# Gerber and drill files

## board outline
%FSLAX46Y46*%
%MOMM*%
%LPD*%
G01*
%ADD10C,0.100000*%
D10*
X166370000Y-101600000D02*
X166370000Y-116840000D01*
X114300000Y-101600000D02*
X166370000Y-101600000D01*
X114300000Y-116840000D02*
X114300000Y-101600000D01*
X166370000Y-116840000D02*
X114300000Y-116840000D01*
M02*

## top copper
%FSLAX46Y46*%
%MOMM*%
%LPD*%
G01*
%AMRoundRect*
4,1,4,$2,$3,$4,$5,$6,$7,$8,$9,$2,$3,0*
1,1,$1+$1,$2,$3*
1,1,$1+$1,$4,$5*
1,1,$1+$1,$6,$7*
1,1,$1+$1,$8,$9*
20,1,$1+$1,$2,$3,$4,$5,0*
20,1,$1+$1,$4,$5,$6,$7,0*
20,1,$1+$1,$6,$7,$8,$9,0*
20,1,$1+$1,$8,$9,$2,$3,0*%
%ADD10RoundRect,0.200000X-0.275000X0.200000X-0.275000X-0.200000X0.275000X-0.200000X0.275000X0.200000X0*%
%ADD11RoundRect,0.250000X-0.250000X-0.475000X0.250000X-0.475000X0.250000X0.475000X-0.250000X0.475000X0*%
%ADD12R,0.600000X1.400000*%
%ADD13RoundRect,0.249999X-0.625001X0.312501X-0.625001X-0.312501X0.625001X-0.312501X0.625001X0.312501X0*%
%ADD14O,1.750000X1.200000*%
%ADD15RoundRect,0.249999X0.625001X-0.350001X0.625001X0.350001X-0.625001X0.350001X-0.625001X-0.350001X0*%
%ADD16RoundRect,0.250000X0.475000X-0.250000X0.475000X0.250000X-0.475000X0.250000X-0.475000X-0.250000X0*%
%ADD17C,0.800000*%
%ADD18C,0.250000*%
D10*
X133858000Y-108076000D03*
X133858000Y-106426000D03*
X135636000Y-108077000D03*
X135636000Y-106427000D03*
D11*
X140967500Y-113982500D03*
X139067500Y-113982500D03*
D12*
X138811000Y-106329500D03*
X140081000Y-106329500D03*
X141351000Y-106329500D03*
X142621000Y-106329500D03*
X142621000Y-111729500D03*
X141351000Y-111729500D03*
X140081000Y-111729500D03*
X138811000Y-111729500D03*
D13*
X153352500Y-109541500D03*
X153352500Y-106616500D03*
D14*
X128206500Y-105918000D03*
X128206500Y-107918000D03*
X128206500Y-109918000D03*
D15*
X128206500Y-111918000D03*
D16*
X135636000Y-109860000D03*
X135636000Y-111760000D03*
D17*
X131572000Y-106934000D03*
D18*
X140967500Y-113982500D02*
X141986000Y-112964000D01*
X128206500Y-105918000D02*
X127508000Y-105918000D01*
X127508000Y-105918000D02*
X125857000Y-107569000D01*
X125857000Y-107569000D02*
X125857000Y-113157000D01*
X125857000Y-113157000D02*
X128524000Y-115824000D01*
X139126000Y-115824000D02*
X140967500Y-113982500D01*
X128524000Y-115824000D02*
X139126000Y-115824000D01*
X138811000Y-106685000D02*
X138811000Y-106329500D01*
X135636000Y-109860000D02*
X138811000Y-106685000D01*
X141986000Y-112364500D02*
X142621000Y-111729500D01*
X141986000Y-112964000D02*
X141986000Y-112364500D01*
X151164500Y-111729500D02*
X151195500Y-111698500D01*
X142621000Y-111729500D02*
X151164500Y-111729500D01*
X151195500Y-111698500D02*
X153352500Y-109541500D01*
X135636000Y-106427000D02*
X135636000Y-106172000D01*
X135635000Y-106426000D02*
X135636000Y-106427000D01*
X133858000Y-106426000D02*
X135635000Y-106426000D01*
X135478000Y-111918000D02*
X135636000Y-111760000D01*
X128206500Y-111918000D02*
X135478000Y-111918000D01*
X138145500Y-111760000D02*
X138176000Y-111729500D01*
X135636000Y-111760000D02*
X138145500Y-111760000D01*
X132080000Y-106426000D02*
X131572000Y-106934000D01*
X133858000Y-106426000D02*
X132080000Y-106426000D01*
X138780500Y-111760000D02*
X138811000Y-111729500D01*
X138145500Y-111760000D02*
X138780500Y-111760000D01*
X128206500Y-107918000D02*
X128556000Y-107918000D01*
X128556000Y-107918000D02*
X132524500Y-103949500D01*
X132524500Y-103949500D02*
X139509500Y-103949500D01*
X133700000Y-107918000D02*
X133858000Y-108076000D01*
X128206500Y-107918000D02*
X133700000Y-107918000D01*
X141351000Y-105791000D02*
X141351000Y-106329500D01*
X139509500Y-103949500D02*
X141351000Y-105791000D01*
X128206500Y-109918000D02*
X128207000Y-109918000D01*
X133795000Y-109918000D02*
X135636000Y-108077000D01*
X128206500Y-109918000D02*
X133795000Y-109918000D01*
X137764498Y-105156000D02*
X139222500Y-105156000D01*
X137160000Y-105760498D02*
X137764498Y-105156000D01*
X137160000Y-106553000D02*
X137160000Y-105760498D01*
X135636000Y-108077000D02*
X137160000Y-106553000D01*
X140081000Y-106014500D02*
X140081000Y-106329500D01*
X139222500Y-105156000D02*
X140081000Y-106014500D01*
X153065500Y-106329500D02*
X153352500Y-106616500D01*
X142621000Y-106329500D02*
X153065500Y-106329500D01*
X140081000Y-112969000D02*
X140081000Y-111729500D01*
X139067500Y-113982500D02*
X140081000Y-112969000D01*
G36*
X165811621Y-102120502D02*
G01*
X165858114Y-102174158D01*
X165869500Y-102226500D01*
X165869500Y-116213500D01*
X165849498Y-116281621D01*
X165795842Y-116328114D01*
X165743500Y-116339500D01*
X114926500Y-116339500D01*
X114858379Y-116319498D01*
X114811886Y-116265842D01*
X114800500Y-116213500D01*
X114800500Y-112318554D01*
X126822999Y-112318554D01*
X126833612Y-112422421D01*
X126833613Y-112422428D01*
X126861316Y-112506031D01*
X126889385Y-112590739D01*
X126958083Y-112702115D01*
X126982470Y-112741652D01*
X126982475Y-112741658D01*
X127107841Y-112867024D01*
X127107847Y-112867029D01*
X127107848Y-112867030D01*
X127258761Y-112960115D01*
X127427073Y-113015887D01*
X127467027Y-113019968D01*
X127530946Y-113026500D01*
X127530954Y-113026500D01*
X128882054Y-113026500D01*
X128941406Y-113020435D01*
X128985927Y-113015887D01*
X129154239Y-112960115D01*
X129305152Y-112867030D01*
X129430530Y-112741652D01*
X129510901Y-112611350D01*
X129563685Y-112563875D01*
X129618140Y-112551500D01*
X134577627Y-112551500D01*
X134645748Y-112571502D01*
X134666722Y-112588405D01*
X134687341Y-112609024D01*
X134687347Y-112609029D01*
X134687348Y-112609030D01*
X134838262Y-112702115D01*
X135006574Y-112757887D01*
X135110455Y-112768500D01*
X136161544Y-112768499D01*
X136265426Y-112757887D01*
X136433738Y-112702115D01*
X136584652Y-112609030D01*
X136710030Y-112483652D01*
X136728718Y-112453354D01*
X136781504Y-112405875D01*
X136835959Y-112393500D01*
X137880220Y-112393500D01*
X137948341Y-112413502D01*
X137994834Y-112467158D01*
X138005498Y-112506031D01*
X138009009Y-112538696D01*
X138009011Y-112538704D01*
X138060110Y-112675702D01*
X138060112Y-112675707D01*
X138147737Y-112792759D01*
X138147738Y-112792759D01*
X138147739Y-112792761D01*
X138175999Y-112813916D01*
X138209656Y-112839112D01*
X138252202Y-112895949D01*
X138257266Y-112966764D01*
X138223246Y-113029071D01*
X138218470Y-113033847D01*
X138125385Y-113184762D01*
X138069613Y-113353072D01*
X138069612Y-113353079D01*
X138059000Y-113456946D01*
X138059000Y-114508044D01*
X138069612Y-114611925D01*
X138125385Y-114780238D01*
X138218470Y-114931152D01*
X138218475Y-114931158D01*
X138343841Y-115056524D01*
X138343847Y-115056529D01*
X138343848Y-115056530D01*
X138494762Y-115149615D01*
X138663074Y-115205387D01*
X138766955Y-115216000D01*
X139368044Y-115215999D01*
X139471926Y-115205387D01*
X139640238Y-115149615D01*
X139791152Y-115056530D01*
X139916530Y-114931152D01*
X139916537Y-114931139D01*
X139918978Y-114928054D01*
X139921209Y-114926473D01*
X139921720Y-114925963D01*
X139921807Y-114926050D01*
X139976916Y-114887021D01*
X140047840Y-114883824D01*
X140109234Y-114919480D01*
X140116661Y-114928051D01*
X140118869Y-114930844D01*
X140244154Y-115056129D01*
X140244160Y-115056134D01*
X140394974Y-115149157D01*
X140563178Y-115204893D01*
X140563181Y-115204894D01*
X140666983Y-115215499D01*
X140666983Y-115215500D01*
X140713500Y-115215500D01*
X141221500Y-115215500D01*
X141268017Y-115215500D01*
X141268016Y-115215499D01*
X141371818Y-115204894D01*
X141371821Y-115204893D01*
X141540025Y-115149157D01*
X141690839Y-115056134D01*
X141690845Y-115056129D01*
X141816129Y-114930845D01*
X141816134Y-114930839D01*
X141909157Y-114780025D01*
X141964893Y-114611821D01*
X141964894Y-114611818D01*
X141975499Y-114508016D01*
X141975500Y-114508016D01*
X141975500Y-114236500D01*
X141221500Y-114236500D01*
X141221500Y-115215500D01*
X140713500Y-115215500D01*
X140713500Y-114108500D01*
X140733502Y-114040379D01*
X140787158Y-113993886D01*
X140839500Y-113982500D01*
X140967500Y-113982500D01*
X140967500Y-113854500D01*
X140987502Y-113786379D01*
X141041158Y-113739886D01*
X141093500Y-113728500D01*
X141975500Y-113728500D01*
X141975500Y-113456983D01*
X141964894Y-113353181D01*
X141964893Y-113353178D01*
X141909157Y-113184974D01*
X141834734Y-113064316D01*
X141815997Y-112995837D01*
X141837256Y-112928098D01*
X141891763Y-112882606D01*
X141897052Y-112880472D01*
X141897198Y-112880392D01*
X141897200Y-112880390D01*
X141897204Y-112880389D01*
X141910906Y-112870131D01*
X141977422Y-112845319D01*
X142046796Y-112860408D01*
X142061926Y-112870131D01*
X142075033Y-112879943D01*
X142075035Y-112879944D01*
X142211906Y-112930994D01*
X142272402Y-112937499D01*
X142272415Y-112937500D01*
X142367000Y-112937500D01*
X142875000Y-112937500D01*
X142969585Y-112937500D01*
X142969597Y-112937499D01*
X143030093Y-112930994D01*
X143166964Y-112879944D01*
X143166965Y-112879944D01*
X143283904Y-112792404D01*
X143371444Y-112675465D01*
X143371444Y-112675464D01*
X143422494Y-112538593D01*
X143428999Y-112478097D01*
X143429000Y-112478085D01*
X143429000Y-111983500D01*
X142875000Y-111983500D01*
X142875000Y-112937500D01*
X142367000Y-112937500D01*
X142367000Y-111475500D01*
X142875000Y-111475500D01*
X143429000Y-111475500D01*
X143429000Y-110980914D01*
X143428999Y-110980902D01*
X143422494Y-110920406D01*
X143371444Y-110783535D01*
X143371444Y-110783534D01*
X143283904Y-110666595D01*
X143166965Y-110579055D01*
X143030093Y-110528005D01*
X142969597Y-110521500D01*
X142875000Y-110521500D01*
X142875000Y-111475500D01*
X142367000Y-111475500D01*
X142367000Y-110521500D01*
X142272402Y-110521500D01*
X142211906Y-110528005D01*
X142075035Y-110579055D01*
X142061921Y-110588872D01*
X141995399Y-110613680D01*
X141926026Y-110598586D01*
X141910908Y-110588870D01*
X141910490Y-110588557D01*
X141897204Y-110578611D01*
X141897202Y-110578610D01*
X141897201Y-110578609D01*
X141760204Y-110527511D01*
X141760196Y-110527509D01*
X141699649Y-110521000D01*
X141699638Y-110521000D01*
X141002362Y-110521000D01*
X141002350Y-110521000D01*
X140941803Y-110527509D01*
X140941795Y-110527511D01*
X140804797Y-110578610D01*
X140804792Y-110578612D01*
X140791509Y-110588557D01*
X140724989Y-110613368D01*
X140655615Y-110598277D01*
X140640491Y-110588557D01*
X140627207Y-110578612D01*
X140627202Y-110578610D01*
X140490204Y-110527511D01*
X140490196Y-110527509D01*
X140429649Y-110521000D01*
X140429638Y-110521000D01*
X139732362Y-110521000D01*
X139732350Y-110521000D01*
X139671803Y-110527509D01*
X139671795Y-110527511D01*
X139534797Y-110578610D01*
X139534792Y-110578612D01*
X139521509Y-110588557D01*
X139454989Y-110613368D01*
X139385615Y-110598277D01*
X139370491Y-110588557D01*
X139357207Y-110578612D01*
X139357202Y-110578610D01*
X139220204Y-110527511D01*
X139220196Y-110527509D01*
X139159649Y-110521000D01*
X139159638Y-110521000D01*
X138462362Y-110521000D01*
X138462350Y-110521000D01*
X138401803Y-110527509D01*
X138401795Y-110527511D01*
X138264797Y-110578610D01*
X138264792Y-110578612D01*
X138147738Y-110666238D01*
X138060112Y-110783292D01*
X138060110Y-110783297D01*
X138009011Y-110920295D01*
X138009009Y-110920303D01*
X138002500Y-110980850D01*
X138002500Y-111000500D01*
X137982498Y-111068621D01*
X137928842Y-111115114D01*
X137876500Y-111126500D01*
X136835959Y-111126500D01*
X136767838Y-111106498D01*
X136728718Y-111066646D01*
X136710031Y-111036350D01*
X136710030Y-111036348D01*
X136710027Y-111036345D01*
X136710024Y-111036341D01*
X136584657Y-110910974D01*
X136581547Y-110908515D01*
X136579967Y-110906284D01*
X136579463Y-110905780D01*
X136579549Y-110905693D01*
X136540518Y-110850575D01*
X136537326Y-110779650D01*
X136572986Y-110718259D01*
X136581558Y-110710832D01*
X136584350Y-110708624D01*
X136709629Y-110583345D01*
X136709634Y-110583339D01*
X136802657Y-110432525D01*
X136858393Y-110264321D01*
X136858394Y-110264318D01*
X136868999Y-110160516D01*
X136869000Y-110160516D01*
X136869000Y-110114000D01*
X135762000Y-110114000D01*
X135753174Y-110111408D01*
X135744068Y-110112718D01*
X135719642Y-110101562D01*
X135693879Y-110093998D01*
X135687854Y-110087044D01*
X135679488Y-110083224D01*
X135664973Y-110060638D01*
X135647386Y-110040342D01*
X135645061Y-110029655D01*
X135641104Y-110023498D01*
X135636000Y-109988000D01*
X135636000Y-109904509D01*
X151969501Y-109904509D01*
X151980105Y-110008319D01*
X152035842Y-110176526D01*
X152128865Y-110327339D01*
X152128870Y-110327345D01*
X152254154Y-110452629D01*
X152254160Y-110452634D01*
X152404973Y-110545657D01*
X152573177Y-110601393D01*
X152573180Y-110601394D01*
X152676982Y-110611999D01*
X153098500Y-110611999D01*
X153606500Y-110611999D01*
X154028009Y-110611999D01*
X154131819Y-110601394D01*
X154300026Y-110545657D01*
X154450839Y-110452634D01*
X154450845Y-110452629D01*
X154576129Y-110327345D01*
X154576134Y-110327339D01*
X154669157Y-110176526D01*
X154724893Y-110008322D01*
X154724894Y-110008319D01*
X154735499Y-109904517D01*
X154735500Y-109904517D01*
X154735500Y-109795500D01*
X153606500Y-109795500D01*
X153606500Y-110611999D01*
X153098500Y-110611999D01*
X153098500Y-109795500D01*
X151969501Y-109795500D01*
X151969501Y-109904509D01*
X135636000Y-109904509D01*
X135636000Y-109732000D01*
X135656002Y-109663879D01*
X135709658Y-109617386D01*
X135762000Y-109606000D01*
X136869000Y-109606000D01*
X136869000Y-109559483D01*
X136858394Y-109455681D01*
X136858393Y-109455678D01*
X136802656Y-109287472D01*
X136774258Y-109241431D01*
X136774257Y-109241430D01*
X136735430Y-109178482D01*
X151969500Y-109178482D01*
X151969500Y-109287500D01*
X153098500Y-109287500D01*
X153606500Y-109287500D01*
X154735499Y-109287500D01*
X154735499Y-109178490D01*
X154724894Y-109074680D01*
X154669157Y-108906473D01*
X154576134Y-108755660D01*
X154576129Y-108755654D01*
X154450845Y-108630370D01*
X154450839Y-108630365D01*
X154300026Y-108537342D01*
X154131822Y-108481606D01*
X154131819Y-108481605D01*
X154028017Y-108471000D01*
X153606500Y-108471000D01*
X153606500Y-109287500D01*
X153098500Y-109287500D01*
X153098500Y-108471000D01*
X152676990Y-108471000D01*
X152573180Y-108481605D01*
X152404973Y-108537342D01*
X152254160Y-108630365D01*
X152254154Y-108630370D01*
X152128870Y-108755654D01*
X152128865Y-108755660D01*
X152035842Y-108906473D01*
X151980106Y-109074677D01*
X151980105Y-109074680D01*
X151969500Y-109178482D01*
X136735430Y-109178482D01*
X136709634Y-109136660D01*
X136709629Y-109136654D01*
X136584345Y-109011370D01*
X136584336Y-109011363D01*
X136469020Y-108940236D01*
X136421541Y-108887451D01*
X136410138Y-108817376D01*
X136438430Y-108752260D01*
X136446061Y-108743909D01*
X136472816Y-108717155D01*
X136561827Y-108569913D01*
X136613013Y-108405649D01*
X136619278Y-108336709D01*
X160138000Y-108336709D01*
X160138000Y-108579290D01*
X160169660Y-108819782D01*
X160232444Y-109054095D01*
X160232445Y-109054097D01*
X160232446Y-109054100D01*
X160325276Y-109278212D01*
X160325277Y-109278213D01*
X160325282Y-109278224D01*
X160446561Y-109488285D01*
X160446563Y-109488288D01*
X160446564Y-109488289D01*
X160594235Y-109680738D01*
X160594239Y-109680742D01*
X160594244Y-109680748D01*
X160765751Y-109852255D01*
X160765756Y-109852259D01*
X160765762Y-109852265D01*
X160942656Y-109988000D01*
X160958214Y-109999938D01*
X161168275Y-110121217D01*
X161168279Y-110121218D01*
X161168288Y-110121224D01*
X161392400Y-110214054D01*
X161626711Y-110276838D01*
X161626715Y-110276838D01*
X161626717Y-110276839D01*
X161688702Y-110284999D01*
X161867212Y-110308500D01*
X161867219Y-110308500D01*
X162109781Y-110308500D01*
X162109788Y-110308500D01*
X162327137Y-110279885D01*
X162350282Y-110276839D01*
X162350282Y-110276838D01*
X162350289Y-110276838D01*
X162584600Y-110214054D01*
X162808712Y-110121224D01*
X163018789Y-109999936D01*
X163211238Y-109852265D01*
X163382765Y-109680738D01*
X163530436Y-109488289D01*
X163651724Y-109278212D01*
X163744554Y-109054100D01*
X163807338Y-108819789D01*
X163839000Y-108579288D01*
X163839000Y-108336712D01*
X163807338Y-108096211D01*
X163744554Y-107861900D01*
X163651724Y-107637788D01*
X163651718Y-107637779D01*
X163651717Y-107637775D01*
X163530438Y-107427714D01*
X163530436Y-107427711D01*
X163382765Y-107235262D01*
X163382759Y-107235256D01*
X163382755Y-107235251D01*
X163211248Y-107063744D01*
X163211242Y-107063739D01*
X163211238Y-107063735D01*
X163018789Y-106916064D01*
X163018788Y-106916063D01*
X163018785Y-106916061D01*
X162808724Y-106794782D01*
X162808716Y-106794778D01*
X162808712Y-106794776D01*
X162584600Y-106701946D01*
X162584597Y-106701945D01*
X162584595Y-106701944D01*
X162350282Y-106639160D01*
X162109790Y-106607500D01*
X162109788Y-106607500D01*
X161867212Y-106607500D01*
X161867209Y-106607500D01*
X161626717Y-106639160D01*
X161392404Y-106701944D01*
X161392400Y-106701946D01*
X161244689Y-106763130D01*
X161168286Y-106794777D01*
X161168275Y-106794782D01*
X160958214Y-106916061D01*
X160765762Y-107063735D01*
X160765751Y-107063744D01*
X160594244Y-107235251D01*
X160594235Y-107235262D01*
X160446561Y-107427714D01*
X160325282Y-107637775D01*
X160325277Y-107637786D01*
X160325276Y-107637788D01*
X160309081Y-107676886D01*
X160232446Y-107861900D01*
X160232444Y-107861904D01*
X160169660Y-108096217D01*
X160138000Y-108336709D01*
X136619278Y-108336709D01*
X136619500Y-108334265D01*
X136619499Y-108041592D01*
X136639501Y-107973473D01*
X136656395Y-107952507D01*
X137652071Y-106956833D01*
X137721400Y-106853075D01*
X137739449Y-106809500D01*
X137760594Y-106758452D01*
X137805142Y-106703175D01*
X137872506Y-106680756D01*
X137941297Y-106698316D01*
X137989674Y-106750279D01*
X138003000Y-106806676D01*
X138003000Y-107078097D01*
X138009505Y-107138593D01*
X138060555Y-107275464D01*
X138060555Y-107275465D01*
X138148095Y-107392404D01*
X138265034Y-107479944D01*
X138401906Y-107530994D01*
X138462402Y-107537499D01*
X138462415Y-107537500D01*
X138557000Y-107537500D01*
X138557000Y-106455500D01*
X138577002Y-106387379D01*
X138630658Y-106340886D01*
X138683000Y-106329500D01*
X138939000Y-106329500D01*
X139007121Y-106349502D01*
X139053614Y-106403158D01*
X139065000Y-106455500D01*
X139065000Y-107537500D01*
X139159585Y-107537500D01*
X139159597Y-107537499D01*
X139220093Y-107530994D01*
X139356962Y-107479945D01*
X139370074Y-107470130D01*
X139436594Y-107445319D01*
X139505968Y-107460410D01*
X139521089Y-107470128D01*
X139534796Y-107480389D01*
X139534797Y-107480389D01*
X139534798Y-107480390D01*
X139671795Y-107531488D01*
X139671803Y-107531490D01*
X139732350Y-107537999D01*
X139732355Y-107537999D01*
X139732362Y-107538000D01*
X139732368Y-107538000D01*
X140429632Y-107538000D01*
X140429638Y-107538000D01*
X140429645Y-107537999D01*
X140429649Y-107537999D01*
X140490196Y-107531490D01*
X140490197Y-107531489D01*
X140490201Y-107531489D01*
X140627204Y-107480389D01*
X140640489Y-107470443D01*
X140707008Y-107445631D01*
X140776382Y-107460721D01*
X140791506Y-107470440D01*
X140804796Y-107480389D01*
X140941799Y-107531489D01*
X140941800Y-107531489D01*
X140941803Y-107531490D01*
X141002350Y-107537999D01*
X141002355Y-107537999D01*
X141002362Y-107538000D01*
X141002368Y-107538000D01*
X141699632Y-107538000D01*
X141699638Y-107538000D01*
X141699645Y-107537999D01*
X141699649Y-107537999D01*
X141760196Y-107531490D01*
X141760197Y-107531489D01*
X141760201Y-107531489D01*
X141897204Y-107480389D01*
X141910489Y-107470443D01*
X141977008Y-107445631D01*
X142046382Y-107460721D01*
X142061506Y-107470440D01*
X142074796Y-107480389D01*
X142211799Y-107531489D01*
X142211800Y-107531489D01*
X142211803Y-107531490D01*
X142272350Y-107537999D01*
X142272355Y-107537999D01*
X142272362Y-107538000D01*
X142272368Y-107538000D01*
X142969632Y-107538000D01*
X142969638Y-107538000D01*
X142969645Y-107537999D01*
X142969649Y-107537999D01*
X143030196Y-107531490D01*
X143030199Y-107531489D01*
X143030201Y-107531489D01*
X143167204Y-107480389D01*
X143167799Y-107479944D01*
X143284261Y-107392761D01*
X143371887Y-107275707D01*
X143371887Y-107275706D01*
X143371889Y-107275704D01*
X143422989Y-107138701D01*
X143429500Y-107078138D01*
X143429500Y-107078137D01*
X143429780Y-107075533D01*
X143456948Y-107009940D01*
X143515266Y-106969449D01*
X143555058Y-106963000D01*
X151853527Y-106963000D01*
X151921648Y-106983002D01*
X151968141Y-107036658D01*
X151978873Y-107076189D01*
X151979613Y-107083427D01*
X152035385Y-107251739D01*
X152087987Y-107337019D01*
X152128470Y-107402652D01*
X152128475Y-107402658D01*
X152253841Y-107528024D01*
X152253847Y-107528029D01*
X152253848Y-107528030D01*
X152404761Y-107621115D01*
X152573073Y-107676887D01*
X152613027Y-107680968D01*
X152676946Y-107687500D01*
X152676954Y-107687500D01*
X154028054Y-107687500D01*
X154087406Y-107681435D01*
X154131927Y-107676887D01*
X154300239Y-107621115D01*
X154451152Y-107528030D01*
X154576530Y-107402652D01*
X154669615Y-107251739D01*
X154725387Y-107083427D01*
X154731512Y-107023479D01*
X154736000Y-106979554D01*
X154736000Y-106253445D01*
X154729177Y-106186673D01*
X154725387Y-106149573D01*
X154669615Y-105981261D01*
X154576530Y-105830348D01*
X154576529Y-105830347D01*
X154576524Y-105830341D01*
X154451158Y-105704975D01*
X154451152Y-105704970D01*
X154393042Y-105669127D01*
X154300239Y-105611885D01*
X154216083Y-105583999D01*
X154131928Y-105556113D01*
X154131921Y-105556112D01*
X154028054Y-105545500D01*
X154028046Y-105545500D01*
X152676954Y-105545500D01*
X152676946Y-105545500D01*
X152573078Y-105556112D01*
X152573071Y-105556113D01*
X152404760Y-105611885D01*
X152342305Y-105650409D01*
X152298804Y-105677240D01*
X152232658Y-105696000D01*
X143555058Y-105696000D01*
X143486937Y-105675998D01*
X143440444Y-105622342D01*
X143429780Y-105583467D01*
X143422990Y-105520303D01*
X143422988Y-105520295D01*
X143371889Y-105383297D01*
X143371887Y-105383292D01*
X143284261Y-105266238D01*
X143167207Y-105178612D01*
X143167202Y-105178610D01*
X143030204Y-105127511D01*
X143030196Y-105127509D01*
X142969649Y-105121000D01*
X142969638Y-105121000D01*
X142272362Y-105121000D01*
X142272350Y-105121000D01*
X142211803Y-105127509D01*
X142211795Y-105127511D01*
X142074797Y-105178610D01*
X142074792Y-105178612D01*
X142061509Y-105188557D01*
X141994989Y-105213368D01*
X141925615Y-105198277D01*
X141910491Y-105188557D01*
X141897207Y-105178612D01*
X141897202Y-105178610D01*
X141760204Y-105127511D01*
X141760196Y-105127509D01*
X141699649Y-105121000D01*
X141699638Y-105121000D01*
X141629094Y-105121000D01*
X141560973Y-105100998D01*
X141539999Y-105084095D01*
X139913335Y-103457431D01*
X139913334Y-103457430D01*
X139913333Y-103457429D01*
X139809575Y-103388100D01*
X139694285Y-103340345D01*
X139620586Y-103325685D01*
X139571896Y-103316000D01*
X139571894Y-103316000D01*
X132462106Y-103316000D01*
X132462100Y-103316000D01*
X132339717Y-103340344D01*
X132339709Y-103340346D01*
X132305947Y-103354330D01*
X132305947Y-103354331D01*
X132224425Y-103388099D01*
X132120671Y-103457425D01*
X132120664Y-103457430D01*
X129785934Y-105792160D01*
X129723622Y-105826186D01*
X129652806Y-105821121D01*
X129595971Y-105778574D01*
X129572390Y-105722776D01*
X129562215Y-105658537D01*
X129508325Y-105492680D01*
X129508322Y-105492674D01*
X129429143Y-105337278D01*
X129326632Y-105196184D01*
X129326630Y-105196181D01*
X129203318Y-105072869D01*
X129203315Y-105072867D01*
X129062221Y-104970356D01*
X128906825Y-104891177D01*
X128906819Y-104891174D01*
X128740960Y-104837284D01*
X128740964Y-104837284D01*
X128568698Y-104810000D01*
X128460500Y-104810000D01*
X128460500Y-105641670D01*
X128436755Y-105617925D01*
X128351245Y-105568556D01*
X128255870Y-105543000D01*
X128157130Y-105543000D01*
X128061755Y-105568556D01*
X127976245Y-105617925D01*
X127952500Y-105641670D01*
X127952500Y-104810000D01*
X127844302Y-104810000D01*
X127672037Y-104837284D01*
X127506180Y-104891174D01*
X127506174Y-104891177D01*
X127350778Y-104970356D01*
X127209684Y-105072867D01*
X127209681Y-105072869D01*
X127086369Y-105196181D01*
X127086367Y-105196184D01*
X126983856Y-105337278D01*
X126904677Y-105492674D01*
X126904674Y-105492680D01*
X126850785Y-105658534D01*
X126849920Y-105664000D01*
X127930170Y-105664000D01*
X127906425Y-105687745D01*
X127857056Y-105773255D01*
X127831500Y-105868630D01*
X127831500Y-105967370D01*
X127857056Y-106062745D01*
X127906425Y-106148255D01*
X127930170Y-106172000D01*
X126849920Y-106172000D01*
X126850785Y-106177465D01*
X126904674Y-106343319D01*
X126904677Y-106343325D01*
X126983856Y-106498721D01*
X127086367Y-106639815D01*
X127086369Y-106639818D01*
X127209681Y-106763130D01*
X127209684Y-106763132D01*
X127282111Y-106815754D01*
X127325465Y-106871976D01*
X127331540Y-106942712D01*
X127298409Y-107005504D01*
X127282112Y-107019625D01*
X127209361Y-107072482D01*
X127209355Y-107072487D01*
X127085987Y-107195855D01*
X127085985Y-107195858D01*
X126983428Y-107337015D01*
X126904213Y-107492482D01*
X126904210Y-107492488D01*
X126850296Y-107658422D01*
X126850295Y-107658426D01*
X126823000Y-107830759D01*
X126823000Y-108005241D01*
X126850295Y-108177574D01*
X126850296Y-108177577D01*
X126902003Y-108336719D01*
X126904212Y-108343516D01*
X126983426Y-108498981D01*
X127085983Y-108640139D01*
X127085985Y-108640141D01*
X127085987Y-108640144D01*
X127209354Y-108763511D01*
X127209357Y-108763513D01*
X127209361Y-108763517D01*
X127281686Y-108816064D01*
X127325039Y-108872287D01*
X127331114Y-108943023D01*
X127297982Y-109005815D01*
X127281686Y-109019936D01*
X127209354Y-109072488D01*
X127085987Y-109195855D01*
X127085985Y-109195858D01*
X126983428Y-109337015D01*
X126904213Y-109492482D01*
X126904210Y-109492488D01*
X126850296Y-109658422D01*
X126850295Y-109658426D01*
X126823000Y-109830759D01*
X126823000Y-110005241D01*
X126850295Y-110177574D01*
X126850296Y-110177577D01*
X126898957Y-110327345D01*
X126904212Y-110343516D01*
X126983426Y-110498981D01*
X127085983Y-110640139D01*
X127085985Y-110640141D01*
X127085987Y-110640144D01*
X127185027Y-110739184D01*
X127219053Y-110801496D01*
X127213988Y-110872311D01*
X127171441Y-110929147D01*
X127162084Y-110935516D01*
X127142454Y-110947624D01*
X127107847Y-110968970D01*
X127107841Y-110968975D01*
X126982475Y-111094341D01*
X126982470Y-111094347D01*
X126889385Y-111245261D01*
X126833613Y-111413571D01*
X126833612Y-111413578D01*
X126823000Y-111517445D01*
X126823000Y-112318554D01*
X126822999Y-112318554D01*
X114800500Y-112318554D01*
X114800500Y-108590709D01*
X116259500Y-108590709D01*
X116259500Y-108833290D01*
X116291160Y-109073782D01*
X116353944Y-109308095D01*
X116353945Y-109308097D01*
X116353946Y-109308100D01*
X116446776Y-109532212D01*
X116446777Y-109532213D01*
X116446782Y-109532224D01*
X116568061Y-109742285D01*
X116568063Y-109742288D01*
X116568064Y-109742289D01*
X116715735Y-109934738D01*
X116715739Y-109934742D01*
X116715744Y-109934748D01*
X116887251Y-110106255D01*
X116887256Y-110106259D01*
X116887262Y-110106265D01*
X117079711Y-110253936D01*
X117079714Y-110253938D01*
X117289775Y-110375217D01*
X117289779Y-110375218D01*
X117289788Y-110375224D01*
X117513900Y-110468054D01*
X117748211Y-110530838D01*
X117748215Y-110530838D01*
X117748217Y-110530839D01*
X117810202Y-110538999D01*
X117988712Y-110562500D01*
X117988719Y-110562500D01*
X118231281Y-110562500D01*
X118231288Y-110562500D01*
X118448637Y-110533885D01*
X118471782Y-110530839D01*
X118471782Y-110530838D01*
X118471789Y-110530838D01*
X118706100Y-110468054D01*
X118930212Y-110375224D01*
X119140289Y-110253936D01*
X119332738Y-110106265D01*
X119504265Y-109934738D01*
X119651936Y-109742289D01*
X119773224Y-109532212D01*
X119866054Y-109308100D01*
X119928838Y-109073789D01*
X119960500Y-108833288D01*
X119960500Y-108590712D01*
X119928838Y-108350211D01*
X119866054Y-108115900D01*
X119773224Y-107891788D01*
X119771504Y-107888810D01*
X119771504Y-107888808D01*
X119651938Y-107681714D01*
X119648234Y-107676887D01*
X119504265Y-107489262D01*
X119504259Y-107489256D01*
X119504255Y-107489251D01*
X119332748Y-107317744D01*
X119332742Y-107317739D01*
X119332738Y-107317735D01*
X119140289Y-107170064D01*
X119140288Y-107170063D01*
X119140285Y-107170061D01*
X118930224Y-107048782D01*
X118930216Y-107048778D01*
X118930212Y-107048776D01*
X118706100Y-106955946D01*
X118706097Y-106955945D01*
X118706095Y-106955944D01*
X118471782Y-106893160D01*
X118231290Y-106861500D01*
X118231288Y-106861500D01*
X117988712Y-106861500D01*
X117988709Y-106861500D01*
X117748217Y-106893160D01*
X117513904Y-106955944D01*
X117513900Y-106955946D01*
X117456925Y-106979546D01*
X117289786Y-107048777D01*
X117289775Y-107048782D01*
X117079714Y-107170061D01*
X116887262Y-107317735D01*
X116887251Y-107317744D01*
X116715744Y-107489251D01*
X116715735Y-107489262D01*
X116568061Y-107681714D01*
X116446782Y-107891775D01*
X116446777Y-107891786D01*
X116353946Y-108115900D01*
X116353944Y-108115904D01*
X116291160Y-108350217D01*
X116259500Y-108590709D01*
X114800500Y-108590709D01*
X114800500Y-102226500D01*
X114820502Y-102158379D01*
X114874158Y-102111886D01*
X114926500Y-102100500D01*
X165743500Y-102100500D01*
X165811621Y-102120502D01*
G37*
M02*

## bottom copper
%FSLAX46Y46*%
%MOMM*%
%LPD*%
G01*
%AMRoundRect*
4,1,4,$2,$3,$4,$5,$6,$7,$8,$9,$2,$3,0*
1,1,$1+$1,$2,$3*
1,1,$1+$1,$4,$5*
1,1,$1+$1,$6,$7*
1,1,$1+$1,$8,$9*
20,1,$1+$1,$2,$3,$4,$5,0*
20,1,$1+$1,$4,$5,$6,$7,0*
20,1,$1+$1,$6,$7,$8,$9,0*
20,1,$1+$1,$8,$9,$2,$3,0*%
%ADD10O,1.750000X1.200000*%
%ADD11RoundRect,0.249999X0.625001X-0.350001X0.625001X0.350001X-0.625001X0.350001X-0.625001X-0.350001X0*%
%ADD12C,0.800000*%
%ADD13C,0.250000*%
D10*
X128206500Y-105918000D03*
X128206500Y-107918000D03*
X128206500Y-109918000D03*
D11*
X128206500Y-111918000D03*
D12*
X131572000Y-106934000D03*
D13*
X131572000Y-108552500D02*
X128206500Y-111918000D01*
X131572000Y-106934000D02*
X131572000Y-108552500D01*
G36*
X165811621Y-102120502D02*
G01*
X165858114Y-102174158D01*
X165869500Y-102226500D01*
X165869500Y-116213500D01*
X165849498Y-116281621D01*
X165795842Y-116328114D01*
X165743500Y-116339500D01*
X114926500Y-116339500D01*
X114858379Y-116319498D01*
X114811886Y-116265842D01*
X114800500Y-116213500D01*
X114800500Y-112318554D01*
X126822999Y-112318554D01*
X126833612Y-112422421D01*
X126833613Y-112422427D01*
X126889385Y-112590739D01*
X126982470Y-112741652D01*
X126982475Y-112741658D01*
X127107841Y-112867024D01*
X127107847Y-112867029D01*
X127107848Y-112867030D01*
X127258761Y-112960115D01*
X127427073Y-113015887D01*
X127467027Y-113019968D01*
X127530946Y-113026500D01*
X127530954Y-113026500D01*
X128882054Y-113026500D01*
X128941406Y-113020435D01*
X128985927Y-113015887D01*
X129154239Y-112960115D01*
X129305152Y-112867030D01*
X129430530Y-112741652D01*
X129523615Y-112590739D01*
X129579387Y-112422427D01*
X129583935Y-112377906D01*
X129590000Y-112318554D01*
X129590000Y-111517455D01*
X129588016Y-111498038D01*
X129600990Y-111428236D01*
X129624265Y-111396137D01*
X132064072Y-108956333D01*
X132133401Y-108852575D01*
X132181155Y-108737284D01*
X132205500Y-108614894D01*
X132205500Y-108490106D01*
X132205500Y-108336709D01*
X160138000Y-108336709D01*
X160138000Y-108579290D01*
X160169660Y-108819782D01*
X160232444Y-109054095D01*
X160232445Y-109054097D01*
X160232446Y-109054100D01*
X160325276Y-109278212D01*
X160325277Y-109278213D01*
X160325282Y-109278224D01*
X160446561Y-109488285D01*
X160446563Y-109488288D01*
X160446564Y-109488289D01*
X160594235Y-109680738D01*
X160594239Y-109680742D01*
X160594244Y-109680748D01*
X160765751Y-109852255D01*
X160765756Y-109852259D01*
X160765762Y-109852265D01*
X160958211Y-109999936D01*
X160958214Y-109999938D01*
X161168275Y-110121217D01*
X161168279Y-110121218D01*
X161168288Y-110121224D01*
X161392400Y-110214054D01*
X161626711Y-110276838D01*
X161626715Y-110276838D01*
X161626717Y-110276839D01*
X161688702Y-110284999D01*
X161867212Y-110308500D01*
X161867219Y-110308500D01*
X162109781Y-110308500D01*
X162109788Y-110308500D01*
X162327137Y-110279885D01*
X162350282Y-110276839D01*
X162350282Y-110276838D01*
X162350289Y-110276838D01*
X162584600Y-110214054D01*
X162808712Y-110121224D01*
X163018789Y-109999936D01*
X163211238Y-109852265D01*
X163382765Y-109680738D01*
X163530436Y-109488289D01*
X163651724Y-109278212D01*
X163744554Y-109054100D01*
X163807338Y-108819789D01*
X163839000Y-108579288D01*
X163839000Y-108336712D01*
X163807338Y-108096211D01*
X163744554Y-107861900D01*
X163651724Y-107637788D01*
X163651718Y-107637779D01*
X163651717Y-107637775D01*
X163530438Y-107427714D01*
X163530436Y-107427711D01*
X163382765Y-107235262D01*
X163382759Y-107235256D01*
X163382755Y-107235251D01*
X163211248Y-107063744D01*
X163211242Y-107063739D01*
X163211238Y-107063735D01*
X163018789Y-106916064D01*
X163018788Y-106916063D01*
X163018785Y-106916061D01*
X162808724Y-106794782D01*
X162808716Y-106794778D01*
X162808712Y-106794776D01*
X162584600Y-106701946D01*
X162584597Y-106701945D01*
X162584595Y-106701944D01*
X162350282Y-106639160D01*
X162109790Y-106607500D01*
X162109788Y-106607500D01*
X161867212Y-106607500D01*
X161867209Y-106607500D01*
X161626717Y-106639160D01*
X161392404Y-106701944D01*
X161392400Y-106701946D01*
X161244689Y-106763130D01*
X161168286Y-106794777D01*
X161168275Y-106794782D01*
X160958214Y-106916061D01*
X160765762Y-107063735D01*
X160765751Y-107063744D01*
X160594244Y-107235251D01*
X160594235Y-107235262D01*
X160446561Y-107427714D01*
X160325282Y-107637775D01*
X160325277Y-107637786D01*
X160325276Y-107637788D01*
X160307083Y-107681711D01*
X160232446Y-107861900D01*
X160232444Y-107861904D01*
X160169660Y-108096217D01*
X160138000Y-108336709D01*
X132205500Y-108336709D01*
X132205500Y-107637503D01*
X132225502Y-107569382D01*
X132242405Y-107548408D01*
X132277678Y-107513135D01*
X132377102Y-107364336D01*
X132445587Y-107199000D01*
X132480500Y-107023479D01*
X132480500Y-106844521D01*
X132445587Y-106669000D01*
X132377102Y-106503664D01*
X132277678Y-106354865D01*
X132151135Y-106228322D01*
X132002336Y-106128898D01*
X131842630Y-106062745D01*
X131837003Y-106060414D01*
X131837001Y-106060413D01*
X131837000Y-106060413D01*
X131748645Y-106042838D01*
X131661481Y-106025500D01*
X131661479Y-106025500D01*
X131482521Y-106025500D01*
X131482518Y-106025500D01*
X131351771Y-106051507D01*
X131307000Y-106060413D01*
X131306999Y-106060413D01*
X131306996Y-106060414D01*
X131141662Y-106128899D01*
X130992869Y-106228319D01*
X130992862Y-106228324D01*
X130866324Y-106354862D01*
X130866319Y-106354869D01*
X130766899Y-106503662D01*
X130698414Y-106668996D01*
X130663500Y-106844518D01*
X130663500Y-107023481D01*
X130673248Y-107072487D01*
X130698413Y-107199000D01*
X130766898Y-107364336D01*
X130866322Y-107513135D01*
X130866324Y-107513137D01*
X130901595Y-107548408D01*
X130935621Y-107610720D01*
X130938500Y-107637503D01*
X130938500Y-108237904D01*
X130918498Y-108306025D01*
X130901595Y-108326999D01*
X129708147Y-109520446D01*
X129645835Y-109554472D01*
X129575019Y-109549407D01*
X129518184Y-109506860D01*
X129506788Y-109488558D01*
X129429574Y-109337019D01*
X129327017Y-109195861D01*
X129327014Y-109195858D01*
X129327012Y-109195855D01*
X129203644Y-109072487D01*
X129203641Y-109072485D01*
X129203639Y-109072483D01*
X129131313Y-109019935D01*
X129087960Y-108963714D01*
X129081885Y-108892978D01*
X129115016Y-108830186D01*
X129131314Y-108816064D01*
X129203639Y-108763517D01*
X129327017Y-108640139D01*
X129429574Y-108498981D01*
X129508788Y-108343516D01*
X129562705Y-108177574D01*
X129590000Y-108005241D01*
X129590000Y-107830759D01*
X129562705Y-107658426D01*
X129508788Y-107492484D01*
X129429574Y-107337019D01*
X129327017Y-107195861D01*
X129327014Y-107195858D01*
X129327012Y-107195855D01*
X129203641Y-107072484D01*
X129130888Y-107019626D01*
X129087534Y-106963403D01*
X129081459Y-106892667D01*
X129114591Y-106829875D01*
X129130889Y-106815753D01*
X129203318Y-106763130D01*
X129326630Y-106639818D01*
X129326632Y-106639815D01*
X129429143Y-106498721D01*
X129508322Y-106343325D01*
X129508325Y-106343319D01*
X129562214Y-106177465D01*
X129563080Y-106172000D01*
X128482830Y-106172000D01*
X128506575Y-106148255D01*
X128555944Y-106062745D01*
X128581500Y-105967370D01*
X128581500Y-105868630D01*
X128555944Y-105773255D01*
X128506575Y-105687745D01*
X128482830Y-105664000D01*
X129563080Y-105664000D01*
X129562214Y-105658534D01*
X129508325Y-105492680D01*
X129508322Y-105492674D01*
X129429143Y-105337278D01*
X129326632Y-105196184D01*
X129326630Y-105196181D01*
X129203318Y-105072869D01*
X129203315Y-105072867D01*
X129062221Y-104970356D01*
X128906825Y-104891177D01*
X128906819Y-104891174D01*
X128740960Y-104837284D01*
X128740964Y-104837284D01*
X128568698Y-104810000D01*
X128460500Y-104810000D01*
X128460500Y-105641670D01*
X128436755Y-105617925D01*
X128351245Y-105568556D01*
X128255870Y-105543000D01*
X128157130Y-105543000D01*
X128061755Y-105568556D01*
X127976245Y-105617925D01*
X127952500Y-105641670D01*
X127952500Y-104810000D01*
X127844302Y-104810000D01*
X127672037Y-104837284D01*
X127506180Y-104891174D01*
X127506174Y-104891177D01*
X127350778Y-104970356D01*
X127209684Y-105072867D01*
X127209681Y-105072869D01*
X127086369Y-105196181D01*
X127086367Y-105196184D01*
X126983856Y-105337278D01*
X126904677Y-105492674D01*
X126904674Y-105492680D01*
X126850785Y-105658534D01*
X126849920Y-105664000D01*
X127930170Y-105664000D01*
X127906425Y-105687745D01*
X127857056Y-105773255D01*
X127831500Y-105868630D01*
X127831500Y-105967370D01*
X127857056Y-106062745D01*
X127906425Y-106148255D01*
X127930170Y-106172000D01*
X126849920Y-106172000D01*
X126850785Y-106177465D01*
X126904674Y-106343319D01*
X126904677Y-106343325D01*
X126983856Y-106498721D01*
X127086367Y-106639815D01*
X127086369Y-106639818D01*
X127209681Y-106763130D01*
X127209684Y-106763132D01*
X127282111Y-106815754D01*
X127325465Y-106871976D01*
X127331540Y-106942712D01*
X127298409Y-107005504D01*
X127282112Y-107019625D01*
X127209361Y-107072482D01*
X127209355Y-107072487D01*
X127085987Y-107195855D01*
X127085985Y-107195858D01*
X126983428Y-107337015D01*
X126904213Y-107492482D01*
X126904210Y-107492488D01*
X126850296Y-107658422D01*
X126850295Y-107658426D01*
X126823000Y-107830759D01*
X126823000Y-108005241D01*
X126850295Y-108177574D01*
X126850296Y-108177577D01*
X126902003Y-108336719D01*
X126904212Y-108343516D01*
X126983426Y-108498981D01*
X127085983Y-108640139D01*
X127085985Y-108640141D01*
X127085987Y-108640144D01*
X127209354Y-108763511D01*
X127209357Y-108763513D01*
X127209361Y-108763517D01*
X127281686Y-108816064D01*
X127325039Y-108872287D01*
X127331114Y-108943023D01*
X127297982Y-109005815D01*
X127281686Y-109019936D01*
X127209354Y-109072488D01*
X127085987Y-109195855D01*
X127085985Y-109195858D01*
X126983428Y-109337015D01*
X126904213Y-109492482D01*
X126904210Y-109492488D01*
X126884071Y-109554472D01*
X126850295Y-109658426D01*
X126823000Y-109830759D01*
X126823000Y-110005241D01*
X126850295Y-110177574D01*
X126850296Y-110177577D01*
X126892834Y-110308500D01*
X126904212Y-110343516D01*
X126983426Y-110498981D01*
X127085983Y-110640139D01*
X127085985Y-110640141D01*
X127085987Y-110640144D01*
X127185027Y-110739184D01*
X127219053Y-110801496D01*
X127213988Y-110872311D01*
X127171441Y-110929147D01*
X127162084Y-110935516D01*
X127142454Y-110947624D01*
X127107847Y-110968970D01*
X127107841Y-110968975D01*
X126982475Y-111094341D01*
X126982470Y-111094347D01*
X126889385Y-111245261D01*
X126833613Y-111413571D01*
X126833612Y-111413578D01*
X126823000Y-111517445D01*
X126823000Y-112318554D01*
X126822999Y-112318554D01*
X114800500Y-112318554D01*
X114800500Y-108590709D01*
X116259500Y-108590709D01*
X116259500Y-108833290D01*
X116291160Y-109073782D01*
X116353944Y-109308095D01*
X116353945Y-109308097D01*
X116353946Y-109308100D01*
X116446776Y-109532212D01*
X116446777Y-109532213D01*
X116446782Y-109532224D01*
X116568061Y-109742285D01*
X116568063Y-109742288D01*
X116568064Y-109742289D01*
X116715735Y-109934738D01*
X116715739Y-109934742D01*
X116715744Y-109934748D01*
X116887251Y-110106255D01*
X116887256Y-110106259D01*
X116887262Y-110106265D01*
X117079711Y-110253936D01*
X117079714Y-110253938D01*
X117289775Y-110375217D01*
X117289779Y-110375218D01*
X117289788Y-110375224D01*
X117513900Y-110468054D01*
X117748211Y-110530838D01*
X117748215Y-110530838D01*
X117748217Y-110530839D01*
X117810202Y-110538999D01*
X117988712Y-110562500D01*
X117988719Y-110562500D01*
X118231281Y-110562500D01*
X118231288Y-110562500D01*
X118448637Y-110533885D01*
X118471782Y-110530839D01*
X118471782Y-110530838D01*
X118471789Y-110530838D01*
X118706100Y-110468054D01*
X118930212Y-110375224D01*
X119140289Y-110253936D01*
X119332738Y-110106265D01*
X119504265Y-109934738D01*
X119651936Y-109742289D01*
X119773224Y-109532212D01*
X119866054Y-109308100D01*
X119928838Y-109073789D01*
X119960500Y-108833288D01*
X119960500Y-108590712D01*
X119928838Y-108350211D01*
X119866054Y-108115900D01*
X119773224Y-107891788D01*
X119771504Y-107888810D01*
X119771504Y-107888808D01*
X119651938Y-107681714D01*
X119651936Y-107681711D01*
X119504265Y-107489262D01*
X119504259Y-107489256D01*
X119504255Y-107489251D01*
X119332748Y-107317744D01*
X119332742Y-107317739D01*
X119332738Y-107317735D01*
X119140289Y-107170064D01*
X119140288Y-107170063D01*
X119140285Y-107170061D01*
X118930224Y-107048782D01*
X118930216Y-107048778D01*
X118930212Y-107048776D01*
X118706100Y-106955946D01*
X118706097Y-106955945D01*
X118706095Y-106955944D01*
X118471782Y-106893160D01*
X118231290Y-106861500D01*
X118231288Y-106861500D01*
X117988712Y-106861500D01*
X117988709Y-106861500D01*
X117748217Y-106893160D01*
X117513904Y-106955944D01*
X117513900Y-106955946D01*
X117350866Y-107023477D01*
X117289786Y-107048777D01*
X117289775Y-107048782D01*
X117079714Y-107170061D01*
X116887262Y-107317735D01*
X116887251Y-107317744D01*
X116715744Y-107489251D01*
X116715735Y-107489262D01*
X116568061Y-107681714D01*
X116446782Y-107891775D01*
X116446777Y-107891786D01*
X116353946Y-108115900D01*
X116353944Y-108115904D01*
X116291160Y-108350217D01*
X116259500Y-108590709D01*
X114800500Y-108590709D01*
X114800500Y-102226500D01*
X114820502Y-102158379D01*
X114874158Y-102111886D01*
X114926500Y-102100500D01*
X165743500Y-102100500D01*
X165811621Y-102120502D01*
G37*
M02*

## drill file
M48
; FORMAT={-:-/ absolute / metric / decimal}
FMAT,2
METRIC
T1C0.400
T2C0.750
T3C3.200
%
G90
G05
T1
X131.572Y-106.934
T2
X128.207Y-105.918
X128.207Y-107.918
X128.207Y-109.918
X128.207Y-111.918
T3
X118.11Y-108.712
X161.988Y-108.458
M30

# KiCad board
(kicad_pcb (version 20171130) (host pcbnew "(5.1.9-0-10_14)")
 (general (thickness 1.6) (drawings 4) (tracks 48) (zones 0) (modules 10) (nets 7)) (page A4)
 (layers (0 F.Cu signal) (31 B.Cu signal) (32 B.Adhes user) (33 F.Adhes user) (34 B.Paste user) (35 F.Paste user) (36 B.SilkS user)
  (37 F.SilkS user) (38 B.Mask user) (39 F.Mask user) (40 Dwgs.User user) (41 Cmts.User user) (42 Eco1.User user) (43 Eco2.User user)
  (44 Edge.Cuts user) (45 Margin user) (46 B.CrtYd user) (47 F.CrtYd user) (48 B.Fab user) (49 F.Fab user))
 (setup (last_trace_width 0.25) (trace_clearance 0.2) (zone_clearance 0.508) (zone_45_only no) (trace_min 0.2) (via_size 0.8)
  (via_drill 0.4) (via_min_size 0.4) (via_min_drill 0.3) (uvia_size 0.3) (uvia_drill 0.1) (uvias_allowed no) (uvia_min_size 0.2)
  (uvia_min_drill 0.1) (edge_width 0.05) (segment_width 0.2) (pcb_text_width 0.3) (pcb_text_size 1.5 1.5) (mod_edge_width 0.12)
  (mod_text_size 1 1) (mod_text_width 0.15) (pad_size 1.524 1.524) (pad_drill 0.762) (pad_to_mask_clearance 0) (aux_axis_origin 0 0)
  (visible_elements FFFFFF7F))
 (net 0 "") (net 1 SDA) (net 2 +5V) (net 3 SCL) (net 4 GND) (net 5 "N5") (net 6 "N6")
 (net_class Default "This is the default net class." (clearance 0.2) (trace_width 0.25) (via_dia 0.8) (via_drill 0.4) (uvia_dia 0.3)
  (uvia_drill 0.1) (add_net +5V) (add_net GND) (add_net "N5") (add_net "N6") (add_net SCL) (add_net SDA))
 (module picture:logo (layer B.Cu) (at 140.97 109.093)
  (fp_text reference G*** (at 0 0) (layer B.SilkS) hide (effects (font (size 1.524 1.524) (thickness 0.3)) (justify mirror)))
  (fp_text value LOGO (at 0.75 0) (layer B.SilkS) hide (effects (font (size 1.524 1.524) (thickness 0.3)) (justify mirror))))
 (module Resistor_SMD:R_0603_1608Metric (layer F.Cu) (at 133.858 107.251 270)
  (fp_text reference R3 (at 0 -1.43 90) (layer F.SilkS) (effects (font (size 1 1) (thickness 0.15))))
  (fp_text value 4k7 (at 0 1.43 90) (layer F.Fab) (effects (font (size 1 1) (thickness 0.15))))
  (pad 2 smd roundrect (at 0.825 0 270) (size 0.8 0.95) (layers F.Cu F.Paste F.Mask) (roundrect_rratio 0.25) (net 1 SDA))
  (pad 1 smd roundrect (at -0.825 0 270) (size 0.8 0.95) (layers F.Cu F.Paste F.Mask) (roundrect_rratio 0.25) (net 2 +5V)))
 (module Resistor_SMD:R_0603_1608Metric (layer F.Cu) (at 135.636 107.252 270)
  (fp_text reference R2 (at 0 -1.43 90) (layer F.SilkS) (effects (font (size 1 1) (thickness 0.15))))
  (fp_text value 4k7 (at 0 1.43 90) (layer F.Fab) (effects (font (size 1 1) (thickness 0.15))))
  (pad 2 smd roundrect (at 0.825 0 270) (size 0.8 0.95) (layers F.Cu F.Paste F.Mask) (roundrect_rratio 0.25) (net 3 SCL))
  (pad 1 smd roundrect (at -0.825 0 270) (size 0.8 0.95) (layers F.Cu F.Paste F.Mask) (roundrect_rratio 0.25) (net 2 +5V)))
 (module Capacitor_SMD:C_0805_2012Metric (layer F.Cu) (at 140.0175 113.9825)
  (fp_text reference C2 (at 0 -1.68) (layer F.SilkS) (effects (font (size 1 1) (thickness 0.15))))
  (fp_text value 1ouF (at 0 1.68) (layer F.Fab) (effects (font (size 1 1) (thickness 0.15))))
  (pad 2 smd roundrect (at 0.95 0) (size 1 1.45) (layers F.Cu F.Paste F.Mask) (roundrect_rratio 0.25) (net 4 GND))
  (pad 1 smd roundrect (at -0.95 0) (size 1 1.45) (layers F.Cu F.Paste F.Mask) (roundrect_rratio 0.25) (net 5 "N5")))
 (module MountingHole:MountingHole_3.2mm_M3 (layer F.Cu) (at 118.11 108.712)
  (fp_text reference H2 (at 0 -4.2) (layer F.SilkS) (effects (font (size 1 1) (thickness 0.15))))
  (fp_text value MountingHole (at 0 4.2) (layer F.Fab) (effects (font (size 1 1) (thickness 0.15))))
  (pad 1 np_thru_hole circle (at 0 0) (size 3.2 3.2) (drill 3.2) (layers *.Cu *.Mask)))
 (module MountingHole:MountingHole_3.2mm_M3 (layer F.Cu) (at 161.9885 108.458)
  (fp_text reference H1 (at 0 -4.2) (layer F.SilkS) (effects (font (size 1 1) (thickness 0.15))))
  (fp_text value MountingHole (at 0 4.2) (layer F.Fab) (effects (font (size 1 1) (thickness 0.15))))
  (pad 1 np_thru_hole circle (at 0 0) (size 3.2 3.2) (drill 3.2) (layers *.Cu *.Mask)))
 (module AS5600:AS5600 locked (layer F.Cu) (at 140.716 109.0295)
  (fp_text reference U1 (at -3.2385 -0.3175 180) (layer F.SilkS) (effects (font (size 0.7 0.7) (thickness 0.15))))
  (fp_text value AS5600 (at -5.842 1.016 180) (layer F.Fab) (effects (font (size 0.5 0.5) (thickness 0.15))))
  (pad 8 smd rect (at -1.905 -2.7) (size 0.6 1.4) (layers F.Cu F.Paste F.Mask) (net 4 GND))
  (pad 7 smd rect (at -0.635 -2.7) (size 0.6 1.4) (layers F.Cu F.Paste F.Mask) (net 3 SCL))
  (pad 6 smd rect (at 0.635 -2.7) (size 0.6 1.4) (layers F.Cu F.Paste F.Mask) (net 1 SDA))
  (pad 5 smd rect (at 1.905 -2.7) (size 0.6 1.4) (layers F.Cu F.Paste F.Mask) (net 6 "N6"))
  (pad 4 smd rect (at 1.905 2.7) (size 0.6 1.4) (layers F.Cu F.Paste F.Mask) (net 4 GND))
  (pad 3 smd rect (at 0.635 2.7) (size 0.6 1.4) (layers F.Cu F.Paste F.Mask))
  (pad 2 smd rect (at -0.635 2.7) (size 0.6 1.4) (layers F.Cu F.Paste F.Mask) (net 5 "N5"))
  (pad 1 smd rect (at -1.905 2.7) (size 0.6 1.4) (layers F.Cu F.Paste F.Mask) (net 2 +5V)))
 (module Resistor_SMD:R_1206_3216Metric (layer F.Cu) (at 153.3525 108.079 270)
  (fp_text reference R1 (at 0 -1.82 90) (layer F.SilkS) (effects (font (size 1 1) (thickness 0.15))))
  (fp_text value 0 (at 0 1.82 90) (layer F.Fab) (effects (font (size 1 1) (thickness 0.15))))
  (pad 2 smd roundrect (at 1.4625 0 270) (size 1.125 1.75) (layers F.Cu F.Paste F.Mask) (roundrect_rratio 0.2222213333333333) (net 4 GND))
  (pad 1 smd roundrect (at -1.4625 0 270) (size 1.125 1.75) (layers F.Cu F.Paste F.Mask) (roundrect_rratio 0.2222213333333333) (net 6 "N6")))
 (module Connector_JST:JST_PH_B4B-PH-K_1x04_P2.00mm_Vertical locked (layer B.Cu) (at 128.2065 111.918 90)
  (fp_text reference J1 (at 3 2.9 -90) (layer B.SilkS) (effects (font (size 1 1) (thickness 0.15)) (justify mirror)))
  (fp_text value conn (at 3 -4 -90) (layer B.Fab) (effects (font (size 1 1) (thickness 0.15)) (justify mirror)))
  (pad 4 thru_hole oval (at 6 0 90) (size 1.2 1.75) (drill 0.75) (layers *.Cu *.Mask) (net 4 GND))
  (pad 3 thru_hole oval (at 4 0 90) (size 1.2 1.75) (drill 0.75) (layers *.Cu *.Mask) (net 1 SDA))
  (pad 2 thru_hole oval (at 2 0 90) (size 1.2 1.75) (drill 0.75) (layers *.Cu *.Mask) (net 3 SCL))
  (pad 1 thru_hole roundrect (at 0 0 90) (size 1.2 1.75) (drill 0.75) (layers *.Cu *.Mask) (roundrect_rratio 0.2083325) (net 2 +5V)))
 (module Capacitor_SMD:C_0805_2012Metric (layer F.Cu) (at 135.636 110.81 90)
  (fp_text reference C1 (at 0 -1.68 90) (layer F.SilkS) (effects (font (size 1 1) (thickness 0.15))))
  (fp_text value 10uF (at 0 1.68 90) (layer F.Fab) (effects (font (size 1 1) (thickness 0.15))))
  (pad 2 smd roundrect (at 0.95 0 90) (size 1 1.45) (layers F.Cu F.Paste F.Mask) (roundrect_rratio 0.25) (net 4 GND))
  (pad 1 smd roundrect (at -0.95 0 90) (size 1 1.45) (layers F.Cu F.Paste F.Mask) (roundrect_rratio 0.25) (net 2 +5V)))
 (gr_line (start 166.37 101.6) (end 166.37 116.84) (layer Edge.Cuts) (width 0.1))
 (gr_line (start 114.3 101.6) (end 166.37 101.6) (layer Edge.Cuts) (width 0.1))
 (gr_line (start 114.3 116.84) (end 114.3 101.6) (layer Edge.Cuts) (width 0.1))
 (gr_line (start 166.37 116.84) (end 114.3 116.84) (layer Edge.Cuts) (width 0.1))
 (segment (start 140.9675 113.9825) (end 141.986 112.964) (width 0.25) (layer F.Cu) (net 4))
 (segment (start 128.2065 105.918) (end 127.508 105.918) (width 0.25) (layer F.Cu) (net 4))
 (segment (start 127.508 105.918) (end 125.857 107.569) (width 0.25) (layer F.Cu) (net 4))
 (segment (start 125.857 107.569) (end 125.857 113.157) (width 0.25) (layer F.Cu) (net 4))
 (segment (start 125.857 113.157) (end 128.524 115.824) (width 0.25) (layer F.Cu) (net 4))
 (segment (start 139.126 115.824) (end 140.9675 113.9825) (width 0.25) (layer F.Cu) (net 4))
 (segment (start 128.524 115.824) (end 139.126 115.824) (width 0.25) (layer F.Cu) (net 4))
 (segment (start 138.811 106.685) (end 138.811 106.3295) (width 0.25) (layer F.Cu) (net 4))
 (segment (start 135.636 109.86) (end 138.811 106.685) (width 0.25) (layer F.Cu) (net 4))
 (segment (start 141.986 112.3645) (end 142.621 111.7295) (width 0.25) (layer F.Cu) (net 4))
 (segment (start 141.986 112.964) (end 141.986 112.3645) (width 0.25) (layer F.Cu) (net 4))
 (segment (start 151.1645 111.7295) (end 151.1955 111.6985) (width 0.25) (layer F.Cu) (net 4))
 (segment (start 142.621 111.7295) (end 151.1645 111.7295) (width 0.25) (layer F.Cu) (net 4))
 (segment (start 151.1955 111.6985) (end 153.3525 109.5415) (width 0.25) (layer F.Cu) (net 4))
 (segment (start 135.636 106.427) (end 135.636 106.172) (width 0.25) (layer F.Cu) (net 2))
 (segment (start 135.635 106.426) (end 135.636 106.427) (width 0.25) (layer F.Cu) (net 2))
 (segment (start 133.858 106.426) (end 135.635 106.426) (width 0.25) (layer F.Cu) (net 2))
 (segment (start 135.478 111.918) (end 135.636 111.76) (width 0.25) (layer F.Cu) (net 2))
 (segment (start 128.2065 111.918) (end 135.478 111.918) (width 0.25) (layer F.Cu) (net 2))
 (segment (start 138.1455 111.76) (end 138.176 111.7295) (width 0.25) (layer F.Cu) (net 2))
 (segment (start 135.636 111.76) (end 138.1455 111.76) (width 0.25) (layer F.Cu) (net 2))
 (via (at 131.572 106.934) (size 0.8) (drill 0.4) (layers F.Cu B.Cu) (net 2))
 (segment (start 132.08 106.426) (end 131.572 106.934) (width 0.25) (layer F.Cu) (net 2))
 (segment (start 133.858 106.426) (end 132.08 106.426) (width 0.25) (layer F.Cu) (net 2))
 (segment (start 131.572 108.5525) (end 128.2065 111.918) (width 0.25) (layer B.Cu) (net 2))
 (segment (start 131.572 106.934) (end 131.572 108.5525) (width 0.25) (layer B.Cu) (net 2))
 (segment (start 138.7805 111.76) (end 138.811 111.7295) (width 0.25) (layer F.Cu) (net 2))
 (segment (start 138.1455 111.76) (end 138.7805 111.76) (width 0.25) (layer F.Cu) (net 2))
 (segment (start 128.2065 107.918) (end 128.556 107.918) (width 0.25) (layer F.Cu) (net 1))
 (segment (start 128.556 107.918) (end 132.5245 103.9495) (width 0.25) (layer F.Cu) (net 1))
 (segment (start 132.5245 103.9495) (end 139.5095 103.9495) (width 0.25) (layer F.Cu) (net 1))
 (segment (start 133.7 107.918) (end 133.858 108.076) (width 0.25) (layer F.Cu) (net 1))
 (segment (start 128.2065 107.918) (end 133.7 107.918) (width 0.25) (layer F.Cu) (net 1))
 (segment (start 141.351 105.791) (end 141.351 106.3295) (width 0.25) (layer F.Cu) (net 1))
 (segment (start 139.5095 103.9495) (end 141.351 105.791) (width 0.25) (layer F.Cu) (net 1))
 (segment (start 128.2065 109.918) (end 128.207 109.918) (width 0.25) (layer F.Cu) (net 3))
 (segment (start 133.795 109.918) (end 135.636 108.077) (width 0.25) (layer F.Cu) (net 3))
 (segment (start 128.2065 109.918) (end 133.795 109.918) (width 0.25) (layer F.Cu) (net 3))
 (segment (start 137.764498 105.156) (end 139.2225 105.156) (width 0.25) (layer F.Cu) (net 3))
 (segment (start 137.16 105.760498) (end 137.764498 105.156) (width 0.25) (layer F.Cu) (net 3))
 (segment (start 137.16 106.553) (end 137.16 105.760498) (width 0.25) (layer F.Cu) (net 3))
 (segment (start 135.636 108.077) (end 137.16 106.553) (width 0.25) (layer F.Cu) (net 3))
 (segment (start 140.081 106.0145) (end 140.081 106.3295) (width 0.25) (layer F.Cu) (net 3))
 (segment (start 139.2225 105.156) (end 140.081 106.0145) (width 0.25) (layer F.Cu) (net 3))
 (segment (start 153.0655 106.3295) (end 153.3525 106.6165) (width 0.25) (layer F.Cu) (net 6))
 (segment (start 142.621 106.3295) (end 153.0655 106.3295) (width 0.25) (layer F.Cu) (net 6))
 (segment (start 140.081 112.969) (end 140.081 111.7295) (width 0.25) (layer F.Cu) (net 5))
 (segment (start 139.0675 113.9825) (end 140.081 112.969) (width 0.25) (layer F.Cu) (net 5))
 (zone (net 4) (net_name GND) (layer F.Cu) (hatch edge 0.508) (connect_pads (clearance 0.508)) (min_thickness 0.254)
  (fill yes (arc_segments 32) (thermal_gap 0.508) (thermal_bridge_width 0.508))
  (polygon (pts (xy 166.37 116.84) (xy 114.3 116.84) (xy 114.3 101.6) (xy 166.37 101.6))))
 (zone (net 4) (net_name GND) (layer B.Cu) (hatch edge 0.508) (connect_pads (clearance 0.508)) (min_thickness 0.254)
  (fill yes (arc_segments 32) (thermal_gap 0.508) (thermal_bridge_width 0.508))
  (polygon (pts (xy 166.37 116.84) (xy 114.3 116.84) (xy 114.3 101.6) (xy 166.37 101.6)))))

